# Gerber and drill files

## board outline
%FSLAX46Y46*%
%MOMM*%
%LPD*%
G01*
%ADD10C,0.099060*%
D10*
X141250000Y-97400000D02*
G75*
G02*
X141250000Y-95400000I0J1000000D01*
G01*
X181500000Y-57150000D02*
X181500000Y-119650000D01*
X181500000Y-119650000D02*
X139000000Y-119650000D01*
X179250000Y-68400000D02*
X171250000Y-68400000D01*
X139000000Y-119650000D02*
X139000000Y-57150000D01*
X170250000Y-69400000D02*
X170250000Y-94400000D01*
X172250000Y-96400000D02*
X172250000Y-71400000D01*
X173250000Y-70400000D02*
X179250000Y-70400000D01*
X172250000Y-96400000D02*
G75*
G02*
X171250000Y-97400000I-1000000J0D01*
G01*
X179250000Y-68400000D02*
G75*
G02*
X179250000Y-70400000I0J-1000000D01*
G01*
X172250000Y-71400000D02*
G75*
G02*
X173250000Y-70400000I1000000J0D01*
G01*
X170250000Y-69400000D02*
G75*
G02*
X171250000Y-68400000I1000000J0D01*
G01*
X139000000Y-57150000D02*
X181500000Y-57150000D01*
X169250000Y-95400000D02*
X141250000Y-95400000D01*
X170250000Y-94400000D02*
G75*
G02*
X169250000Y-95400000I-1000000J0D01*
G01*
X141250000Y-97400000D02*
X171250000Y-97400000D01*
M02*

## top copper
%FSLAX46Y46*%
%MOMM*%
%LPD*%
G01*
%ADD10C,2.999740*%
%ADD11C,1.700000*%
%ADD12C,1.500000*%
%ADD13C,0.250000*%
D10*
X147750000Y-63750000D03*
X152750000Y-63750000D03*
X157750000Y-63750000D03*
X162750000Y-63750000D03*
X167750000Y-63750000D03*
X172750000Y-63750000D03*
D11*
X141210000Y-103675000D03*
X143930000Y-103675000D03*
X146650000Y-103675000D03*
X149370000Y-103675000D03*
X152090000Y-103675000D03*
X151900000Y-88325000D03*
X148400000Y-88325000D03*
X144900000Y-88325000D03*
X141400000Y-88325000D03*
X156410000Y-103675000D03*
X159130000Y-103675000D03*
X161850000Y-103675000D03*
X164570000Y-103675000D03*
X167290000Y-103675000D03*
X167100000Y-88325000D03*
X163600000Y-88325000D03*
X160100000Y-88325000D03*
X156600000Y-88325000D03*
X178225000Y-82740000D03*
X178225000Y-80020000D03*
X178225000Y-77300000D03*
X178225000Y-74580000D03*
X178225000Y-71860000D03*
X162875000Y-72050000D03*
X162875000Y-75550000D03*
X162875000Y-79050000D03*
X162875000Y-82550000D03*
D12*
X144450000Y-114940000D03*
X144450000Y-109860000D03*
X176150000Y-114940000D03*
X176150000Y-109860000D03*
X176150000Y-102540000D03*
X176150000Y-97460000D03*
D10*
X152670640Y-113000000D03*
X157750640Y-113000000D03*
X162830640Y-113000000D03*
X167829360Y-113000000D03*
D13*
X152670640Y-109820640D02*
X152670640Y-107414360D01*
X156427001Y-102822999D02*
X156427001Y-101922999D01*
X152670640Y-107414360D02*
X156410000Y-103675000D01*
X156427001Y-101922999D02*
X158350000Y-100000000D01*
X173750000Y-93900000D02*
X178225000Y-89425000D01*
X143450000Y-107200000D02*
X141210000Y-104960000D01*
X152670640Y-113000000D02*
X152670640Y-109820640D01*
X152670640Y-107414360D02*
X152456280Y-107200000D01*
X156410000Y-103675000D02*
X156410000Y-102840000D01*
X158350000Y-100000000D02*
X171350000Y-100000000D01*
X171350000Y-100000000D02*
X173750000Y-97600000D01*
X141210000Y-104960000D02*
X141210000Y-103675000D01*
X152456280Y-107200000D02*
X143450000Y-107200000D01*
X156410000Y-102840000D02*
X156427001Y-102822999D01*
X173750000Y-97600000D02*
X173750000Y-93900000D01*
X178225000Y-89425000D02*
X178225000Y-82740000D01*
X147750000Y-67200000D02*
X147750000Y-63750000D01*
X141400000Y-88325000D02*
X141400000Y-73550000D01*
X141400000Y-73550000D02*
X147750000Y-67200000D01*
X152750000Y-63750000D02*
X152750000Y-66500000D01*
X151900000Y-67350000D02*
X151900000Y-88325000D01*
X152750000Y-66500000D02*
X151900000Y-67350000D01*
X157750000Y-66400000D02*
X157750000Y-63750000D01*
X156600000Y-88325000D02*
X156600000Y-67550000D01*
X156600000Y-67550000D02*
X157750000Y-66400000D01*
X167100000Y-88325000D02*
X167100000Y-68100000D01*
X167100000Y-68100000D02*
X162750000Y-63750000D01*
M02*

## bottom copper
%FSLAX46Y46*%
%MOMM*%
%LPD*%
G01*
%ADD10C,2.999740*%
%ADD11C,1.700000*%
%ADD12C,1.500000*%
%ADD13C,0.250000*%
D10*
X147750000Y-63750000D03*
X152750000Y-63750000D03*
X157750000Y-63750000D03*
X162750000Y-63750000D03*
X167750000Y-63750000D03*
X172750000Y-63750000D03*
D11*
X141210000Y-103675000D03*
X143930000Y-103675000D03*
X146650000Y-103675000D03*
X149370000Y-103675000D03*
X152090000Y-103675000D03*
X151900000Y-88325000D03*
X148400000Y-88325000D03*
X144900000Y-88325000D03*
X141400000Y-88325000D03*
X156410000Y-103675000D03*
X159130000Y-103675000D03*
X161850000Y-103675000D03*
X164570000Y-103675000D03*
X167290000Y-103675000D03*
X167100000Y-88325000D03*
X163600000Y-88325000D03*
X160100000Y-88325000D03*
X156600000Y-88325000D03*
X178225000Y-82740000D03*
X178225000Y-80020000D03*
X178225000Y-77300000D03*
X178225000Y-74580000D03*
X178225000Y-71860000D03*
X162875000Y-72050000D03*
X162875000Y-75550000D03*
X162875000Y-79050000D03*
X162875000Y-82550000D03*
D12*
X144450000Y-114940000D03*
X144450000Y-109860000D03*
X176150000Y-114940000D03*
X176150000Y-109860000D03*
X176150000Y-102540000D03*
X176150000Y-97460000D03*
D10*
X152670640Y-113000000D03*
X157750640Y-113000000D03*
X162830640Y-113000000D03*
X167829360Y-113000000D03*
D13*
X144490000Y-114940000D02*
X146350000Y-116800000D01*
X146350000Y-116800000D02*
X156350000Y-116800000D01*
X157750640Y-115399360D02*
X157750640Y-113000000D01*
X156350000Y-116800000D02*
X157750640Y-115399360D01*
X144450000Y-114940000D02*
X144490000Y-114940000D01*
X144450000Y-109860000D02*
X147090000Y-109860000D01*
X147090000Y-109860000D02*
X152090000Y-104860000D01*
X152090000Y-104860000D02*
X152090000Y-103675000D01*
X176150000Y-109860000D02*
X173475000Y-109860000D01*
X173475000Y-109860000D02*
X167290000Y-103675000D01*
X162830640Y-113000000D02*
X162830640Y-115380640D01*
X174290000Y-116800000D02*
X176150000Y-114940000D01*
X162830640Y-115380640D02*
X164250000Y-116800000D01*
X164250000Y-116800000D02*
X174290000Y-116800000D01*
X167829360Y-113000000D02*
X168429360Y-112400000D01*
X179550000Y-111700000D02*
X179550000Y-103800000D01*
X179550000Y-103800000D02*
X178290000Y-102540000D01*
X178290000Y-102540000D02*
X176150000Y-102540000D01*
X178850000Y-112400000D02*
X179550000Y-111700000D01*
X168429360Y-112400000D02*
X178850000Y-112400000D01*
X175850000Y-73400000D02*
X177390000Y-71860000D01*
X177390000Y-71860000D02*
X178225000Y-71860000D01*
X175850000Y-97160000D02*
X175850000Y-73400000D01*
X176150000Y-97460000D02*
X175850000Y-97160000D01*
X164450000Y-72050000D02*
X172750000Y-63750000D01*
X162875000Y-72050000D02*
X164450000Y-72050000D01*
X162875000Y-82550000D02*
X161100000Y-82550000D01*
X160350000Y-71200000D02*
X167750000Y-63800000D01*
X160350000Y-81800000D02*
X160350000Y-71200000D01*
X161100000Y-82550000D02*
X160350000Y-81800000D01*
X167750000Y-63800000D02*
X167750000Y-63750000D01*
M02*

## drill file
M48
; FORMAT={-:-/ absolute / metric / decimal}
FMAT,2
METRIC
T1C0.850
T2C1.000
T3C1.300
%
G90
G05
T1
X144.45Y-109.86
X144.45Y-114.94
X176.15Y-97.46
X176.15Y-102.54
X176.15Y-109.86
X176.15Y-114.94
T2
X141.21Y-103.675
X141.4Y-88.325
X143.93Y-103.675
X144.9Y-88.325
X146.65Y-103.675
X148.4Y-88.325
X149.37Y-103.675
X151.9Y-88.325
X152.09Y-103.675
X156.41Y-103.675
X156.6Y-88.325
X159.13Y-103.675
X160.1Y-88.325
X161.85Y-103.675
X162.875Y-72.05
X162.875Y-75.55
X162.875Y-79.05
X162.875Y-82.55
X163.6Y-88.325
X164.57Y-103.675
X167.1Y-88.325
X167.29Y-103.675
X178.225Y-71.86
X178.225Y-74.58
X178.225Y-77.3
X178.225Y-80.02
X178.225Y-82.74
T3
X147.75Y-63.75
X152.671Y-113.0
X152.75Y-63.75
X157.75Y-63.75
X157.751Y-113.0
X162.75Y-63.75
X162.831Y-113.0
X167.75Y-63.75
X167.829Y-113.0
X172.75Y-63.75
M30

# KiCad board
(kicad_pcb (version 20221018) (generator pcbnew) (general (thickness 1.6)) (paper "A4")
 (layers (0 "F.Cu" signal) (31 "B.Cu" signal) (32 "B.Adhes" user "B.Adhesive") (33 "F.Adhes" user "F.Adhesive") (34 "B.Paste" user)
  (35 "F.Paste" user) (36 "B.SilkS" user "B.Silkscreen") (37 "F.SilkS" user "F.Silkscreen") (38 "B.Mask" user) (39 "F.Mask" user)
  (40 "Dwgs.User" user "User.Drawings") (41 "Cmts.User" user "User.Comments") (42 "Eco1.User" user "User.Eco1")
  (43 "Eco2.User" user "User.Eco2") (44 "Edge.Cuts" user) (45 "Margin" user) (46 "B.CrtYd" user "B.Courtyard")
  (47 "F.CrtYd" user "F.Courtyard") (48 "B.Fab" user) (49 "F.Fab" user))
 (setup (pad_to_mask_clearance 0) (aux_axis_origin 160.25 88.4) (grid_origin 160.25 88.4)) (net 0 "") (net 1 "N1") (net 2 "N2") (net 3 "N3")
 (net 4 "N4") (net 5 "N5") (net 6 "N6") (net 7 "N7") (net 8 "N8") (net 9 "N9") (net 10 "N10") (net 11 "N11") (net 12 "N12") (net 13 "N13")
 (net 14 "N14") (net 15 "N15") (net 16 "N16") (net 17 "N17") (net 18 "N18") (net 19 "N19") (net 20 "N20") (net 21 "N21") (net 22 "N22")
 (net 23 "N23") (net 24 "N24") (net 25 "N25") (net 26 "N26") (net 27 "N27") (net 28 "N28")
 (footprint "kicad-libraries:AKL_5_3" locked (layer "F.Cu") (at 152.75 63.75)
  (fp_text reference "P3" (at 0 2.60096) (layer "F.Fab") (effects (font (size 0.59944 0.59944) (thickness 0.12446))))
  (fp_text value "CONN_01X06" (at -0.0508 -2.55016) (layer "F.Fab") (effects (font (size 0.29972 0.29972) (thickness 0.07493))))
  (pad "1" thru_hole circle locked (at -5 0) (size 2.99974 2.99974) (drill 1.30048) (layers "*.Cu" "*.Mask" "F.SilkS") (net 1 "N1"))
  (pad "2" thru_hole circle locked (at 0 0) (size 2.99974 2.99974) (drill 1.30048) (layers "*.Cu" "*.Mask" "F.SilkS") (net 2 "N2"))
  (pad "3" thru_hole circle locked (at 5 0) (size 2.99974 2.99974) (drill 1.30048) (layers "*.Cu" "*.Mask" "F.SilkS") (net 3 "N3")))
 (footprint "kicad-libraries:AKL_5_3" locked (layer "F.Cu") (at 167.75 63.75)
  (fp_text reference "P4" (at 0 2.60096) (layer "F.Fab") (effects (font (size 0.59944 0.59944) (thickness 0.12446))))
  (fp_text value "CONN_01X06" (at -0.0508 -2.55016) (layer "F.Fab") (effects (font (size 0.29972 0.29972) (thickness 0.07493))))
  (pad "1" thru_hole circle locked (at -5 0) (size 2.99974 2.99974) (drill 1.30048) (layers "*.Cu" "*.Mask" "F.SilkS") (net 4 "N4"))
  (pad "2" thru_hole circle locked (at 0 0) (size 2.99974 2.99974) (drill 1.30048) (layers "*.Cu" "*.Mask" "F.SilkS") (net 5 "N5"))
  (pad "3" thru_hole circle locked (at 5 0) (size 2.99974 2.99974) (drill 1.30048) (layers "*.Cu" "*.Mask" "F.SilkS") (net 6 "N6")))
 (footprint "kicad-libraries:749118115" (layer "F.Cu") (at 146.65 96)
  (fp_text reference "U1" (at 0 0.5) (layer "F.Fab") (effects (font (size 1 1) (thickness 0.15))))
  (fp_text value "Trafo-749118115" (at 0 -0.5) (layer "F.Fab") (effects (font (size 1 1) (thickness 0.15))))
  (pad "1" thru_hole circle (at -5.44 7.675) (size 1.7 1.7) (drill 1) (layers "*.Cu" "*.Mask") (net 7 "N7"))
  (pad "2" thru_hole circle (at -2.72 7.675) (size 1.7 1.7) (drill 1) (layers "*.Cu" "*.Mask") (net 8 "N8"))
  (pad "3" thru_hole circle (at 0 7.675) (size 1.7 1.7) (drill 1) (layers "*.Cu" "*.Mask") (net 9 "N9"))
  (pad "4" thru_hole circle (at 2.72 7.675) (size 1.7 1.7) (drill 1) (layers "*.Cu" "*.Mask") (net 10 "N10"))
  (pad "5" thru_hole circle (at 5.44 7.675) (size 1.7 1.7) (drill 1) (layers "*.Cu" "*.Mask") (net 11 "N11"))
  (pad "6" thru_hole circle (at 5.25 -7.675) (size 1.7 1.7) (drill 1) (layers "*.Cu" "*.Mask") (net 2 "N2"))
  (pad "7" thru_hole circle (at 1.75 -7.675) (size 1.7 1.7) (drill 1) (layers "*.Cu" "*.Mask") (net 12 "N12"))
  (pad "8" thru_hole circle (at -1.75 -7.675) (size 1.7 1.7) (drill 1) (layers "*.Cu" "*.Mask") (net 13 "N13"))
  (pad "9" thru_hole circle (at -5.25 -7.675) (size 1.7 1.7) (drill 1) (layers "*.Cu" "*.Mask") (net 1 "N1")))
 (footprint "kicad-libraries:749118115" (layer "F.Cu") (at 161.85 96)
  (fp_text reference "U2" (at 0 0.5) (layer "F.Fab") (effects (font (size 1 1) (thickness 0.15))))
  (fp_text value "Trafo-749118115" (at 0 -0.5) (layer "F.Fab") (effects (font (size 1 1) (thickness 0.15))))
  (pad "1" thru_hole circle (at -5.44 7.675) (size 1.7 1.7) (drill 1) (layers "*.Cu" "*.Mask") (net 7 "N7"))
  (pad "2" thru_hole circle (at -2.72 7.675) (size 1.7 1.7) (drill 1) (layers "*.Cu" "*.Mask") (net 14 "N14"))
  (pad "3" thru_hole circle (at 0 7.675) (size 1.7 1.7) (drill 1) (layers "*.Cu" "*.Mask") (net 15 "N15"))
  (pad "4" thru_hole circle (at 2.72 7.675) (size 1.7 1.7) (drill 1) (layers "*.Cu" "*.Mask") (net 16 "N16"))
  (pad "5" thru_hole circle (at 5.44 7.675) (size 1.7 1.7) (drill 1) (layers "*.Cu" "*.Mask") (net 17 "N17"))
  (pad "6" thru_hole circle (at 5.25 -7.675) (size 1.7 1.7) (drill 1) (layers "*.Cu" "*.Mask") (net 4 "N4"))
  (pad "7" thru_hole circle (at 1.75 -7.675) (size 1.7 1.7) (drill 1) (layers "*.Cu" "*.Mask") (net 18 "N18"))
  (pad "8" thru_hole circle (at -1.75 -7.675) (size 1.7 1.7) (drill 1) (layers "*.Cu" "*.Mask") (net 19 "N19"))
  (pad "9" thru_hole circle (at -5.25 -7.675) (size 1.7 1.7) (drill 1) (layers "*.Cu" "*.Mask") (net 3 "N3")))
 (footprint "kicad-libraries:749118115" (layer "F.Cu") (at 170.55 77.3 90)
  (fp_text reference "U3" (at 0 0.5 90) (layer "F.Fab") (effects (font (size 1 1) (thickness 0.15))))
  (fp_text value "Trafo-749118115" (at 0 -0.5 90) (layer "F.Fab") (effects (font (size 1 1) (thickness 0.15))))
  (pad "1" thru_hole circle (at -5.44 7.675 90) (size 1.7 1.7) (drill 1) (layers "*.Cu" "*.Mask") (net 7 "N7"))
  (pad "2" thru_hole circle (at -2.72 7.675 90) (size 1.7 1.7) (drill 1) (layers "*.Cu" "*.Mask") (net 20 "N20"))
  (pad "3" thru_hole circle (at 0 7.675 90) (size 1.7 1.7) (drill 1) (layers "*.Cu" "*.Mask") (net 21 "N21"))
  (pad "4" thru_hole circle (at 2.72 7.675 90) (size 1.7 1.7) (drill 1) (layers "*.Cu" "*.Mask") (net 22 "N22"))
  (pad "5" thru_hole circle (at 5.44 7.675 90) (size 1.7 1.7) (drill 1) (layers "*.Cu" "*.Mask") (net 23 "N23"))
  (pad "6" thru_hole circle (at 5.25 -7.675 90) (size 1.7 1.7) (drill 1) (layers "*.Cu" "*.Mask") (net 6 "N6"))
  (pad "7" thru_hole circle (at 1.75 -7.675 90) (size 1.7 1.7) (drill 1) (layers "*.Cu" "*.Mask") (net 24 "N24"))
  (pad "8" thru_hole circle (at -1.75 -7.675 90) (size 1.7 1.7) (drill 1) (layers "*.Cu" "*.Mask") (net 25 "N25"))
  (pad "9" thru_hole circle (at -5.25 -7.675 90) (size 1.7 1.7) (drill 1) (layers "*.Cu" "*.Mask") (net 5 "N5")))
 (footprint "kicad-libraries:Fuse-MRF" (layer "F.Cu") (at 144.45 112.4 90)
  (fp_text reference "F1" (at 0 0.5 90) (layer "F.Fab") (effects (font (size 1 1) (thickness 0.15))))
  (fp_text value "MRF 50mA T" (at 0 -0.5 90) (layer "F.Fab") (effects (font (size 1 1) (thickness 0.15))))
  (pad "1" thru_hole circle (at -2.54 0 90) (size 1.5 1.5) (drill 0.85) (layers "*.Cu" "*.Mask") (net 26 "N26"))
  (pad "2" thru_hole circle (at 2.54 0 90) (size 1.5 1.5) (drill 0.85) (layers "*.Cu" "*.Mask") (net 11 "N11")))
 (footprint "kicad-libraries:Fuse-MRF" (layer "F.Cu") (at 176.15 112.4 90)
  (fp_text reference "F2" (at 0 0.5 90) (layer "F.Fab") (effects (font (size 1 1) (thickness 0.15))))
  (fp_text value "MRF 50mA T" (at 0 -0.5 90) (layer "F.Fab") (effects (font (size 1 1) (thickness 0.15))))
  (pad "1" thru_hole circle (at -2.54 0 90) (size 1.5 1.5) (drill 0.85) (layers "*.Cu" "*.Mask") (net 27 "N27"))
  (pad "2" thru_hole circle (at 2.54 0 90) (size 1.5 1.5) (drill 0.85) (layers "*.Cu" "*.Mask") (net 17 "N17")))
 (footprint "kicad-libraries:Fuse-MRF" (layer "F.Cu") (at 176.15 100 90)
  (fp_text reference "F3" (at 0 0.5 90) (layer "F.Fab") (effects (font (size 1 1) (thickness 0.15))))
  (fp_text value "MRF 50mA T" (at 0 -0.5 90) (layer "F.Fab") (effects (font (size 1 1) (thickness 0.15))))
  (pad "1" thru_hole circle (at -2.54 0 90) (size 1.5 1.5) (drill 0.85) (layers "*.Cu" "*.Mask") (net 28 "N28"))
  (pad "2" thru_hole circle (at 2.54 0 90) (size 1.5 1.5) (drill 0.85) (layers "*.Cu" "*.Mask") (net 23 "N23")))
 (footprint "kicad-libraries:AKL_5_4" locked (layer "F.Cu") (at 160.25 113 180)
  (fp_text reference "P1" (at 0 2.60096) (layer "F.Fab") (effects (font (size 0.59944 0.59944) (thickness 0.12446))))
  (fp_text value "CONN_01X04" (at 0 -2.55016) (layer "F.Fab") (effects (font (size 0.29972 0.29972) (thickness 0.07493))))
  (pad "1" thru_hole circle locked (at 7.57936 0 180) (size 2.99974 2.99974) (drill 1.30048) (layers "*.Cu" "*.Mask" "F.SilkS") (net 7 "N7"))
  (pad "2" thru_hole circle locked (at 2.49936 0 180) (size 2.99974 2.99974) (drill 1.30048) (layers "*.Cu" "*.Mask" "F.SilkS")
   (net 26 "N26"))
  (pad "3" thru_hole circle locked (at -2.58064 0 180) (size 2.99974 2.99974) (drill 1.30048) (layers "*.Cu" "*.Mask" "F.SilkS")
   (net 27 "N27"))
  (pad "4" thru_hole circle locked (at -7.57936 0 180) (size 2.99974 2.99974) (drill 1.30048) (layers "*.Cu" "*.Mask" "F.SilkS")
   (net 28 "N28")))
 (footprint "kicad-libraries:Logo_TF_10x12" (layer "F.Cu") (at 149.25 74.4)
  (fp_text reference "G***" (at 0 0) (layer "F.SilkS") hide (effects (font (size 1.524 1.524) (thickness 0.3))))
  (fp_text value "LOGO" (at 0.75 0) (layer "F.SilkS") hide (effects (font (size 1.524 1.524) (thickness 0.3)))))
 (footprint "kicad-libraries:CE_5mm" (layer "B.Cu") (at 148.95 73.1 180)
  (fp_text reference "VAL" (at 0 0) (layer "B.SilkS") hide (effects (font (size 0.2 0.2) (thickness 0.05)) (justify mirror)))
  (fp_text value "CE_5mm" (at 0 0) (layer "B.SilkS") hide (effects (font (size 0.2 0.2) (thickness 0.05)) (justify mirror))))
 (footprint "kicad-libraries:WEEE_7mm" (layer "B.Cu") (at 148.85 80.5 180)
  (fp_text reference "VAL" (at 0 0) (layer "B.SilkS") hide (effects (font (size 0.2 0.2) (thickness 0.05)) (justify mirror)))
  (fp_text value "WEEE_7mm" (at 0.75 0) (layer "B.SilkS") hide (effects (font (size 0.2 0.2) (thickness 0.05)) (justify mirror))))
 (gr_arc (start 141.25 97.4) (mid 140.25 96.4) (end 141.25 95.4) (stroke (width 0.09906) (type solid)) (layer "Edge.Cuts"))
 (gr_line (start 181.5 57.15) (end 181.5 119.65) (stroke (width 0.09906) (type solid)) (layer "Edge.Cuts"))
 (gr_line (start 181.5 119.65) (end 139 119.65) (stroke (width 0.09906) (type solid)) (layer "Edge.Cuts"))
 (gr_line (start 179.25 68.4) (end 171.25 68.4) (stroke (width 0.09906) (type solid)) (layer "Edge.Cuts"))
 (gr_line (start 139 119.65) (end 139 57.15) (stroke (width 0.09906) (type solid)) (layer "Edge.Cuts"))
 (gr_line (start 170.25 69.4) (end 170.25 94.4) (stroke (width 0.09906) (type solid)) (layer "Edge.Cuts"))
 (gr_line (start 172.25 96.4) (end 172.25 71.4) (stroke (width 0.09906) (type solid)) (layer "Edge.Cuts"))
 (gr_line (start 173.25 70.4) (end 179.25 70.4) (stroke (width 0.09906) (type solid)) (layer "Edge.Cuts"))
 (gr_arc (start 172.25 96.4) (mid 171.957107 97.107107) (end 171.25 97.4) (stroke (width 0.09906) (type solid)) (layer "Edge.Cuts"))
 (gr_arc (start 179.25 68.4) (mid 180.25 69.4) (end 179.25 70.4) (stroke (width 0.09906) (type solid)) (layer "Edge.Cuts"))
 (gr_arc (start 172.25 71.4) (mid 172.542893 70.692893) (end 173.25 70.4) (stroke (width 0.09906) (type solid)) (layer "Edge.Cuts"))
 (gr_arc (start 170.25 69.4) (mid 170.542893 68.692893) (end 171.25 68.4) (stroke (width 0.09906) (type solid)) (layer "Edge.Cuts"))
 (gr_line (start 139 57.15) (end 181.5 57.15) (stroke (width 0.09906) (type solid)) (layer "Edge.Cuts"))
 (gr_line (start 169.25 95.4) (end 141.25 95.4) (stroke (width 0.09906) (type solid)) (layer "Edge.Cuts"))
 (gr_arc (start 170.25 94.4) (mid 169.957107 95.107107) (end 169.25 95.4) (stroke (width 0.09906) (type solid)) (layer "Edge.Cuts"))
 (gr_line (start 141.25 97.4) (end 171.25 97.4) (stroke (width 0.09906) (type solid)) (layer "Edge.Cuts"))
 (segment (start 144.49 114.94) (end 146.35 116.8) (width 0.25) (layer "B.Cu") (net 26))
 (segment (start 146.35 116.8) (end 156.35 116.8) (width 0.25) (layer "B.Cu") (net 26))
 (segment (start 157.75064 115.39936) (end 157.75064 113) (width 0.25) (layer "B.Cu") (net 26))
 (segment (start 156.35 116.8) (end 157.75064 115.39936) (width 0.25) (layer "B.Cu") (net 26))
 (segment (start 144.45 114.94) (end 144.49 114.94) (width 0.25) (layer "B.Cu") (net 26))
 (segment (start 144.45 109.86) (end 147.09 109.86) (width 0.25) (layer "B.Cu") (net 11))
 (segment (start 147.09 109.86) (end 152.09 104.86) (width 0.25) (layer "B.Cu") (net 11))
 (segment (start 152.09 104.86) (end 152.09 103.675) (width 0.25) (layer "B.Cu") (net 11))
 (segment (start 176.15 109.86) (end 173.475 109.86) (width 0.25) (layer "B.Cu") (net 17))
 (segment (start 173.475 109.86) (end 167.29 103.675) (width 0.25) (layer "B.Cu") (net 17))
 (segment (start 162.83064 113) (end 162.83064 115.38064) (width 0.25) (layer "B.Cu") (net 27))
 (segment (start 174.29 116.8) (end 176.15 114.94) (width 0.25) (layer "B.Cu") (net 27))
 (segment (start 162.83064 115.38064) (end 164.25 116.8) (width 0.25) (layer "B.Cu") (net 27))
 (segment (start 164.25 116.8) (end 174.29 116.8) (width 0.25) (layer "B.Cu") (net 27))
 (segment (start 167.82936 113) (end 168.42936 112.4) (width 0.25) (layer "B.Cu") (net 28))
 (segment (start 179.55 111.7) (end 179.55 103.8) (width 0.25) (layer "B.Cu") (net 28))
 (segment (start 179.55 103.8) (end 178.29 102.54) (width 0.25) (layer "B.Cu") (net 28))
 (segment (start 178.29 102.54) (end 176.15 102.54) (width 0.25) (layer "B.Cu") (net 28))
 (segment (start 178.85 112.4) (end 179.55 111.7) (width 0.25) (layer "B.Cu") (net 28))
 (segment (start 168.42936 112.4) (end 178.85 112.4) (width 0.25) (layer "B.Cu") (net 28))
 (segment (start 175.85 73.4) (end 177.39 71.86) (width 0.25) (layer "B.Cu") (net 23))
 (segment (start 177.39 71.86) (end 178.225 71.86) (width 0.25) (layer "B.Cu") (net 23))
 (segment (start 175.85 97.16) (end 175.85 73.4) (width 0.25) (layer "B.Cu") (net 23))
 (segment (start 176.15 97.46) (end 175.85 97.16) (width 0.25) (layer "B.Cu") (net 23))
 (segment (start 152.67064 109.82064) (end 152.67064 107.41436) (width 0.25) (layer "F.Cu") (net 7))
 (segment (start 156.427001 102.822999) (end 156.427001 101.922999) (width 0.25) (layer "F.Cu") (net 7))
 (segment (start 152.67064 107.41436) (end 156.41 103.675) (width 0.25) (layer "F.Cu") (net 7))
 (segment (start 156.427001 101.922999) (end 158.35 100) (width 0.25) (layer "F.Cu") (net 7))
 (segment (start 173.75 93.9) (end 178.225 89.425) (width 0.25) (layer "F.Cu") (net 7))
 (segment (start 143.45 107.2) (end 141.21 104.96) (width 0.25) (layer "F.Cu") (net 7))
 (segment (start 152.67064 113) (end 152.67064 109.82064) (width 0.25) (layer "F.Cu") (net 7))
 (segment (start 152.67064 107.41436) (end 152.45628 107.2) (width 0.25) (layer "F.Cu") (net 7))
 (segment (start 156.41 103.675) (end 156.41 102.84) (width 0.25) (layer "F.Cu") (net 7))
 (segment (start 158.35 100) (end 171.35 100) (width 0.25) (layer "F.Cu") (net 7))
 (segment (start 171.35 100) (end 173.75 97.6) (width 0.25) (layer "F.Cu") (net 7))
 (segment (start 141.21 104.96) (end 141.21 103.675) (width 0.25) (layer "F.Cu") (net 7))
 (segment (start 152.45628 107.2) (end 143.45 107.2) (width 0.25) (layer "F.Cu") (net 7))
 (segment (start 156.41 102.84) (end 156.427001 102.822999) (width 0.25) (layer "F.Cu") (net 7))
 (segment (start 173.75 97.6) (end 173.75 93.9) (width 0.25) (layer "F.Cu") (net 7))
 (segment (start 178.225 89.425) (end 178.225 82.74) (width 0.25) (layer "F.Cu") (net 7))
 (segment (start 147.75 67.2) (end 147.75 63.75) (width 0.25) (layer "F.Cu") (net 1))
 (segment (start 141.4 88.325) (end 141.4 73.55) (width 0.25) (layer "F.Cu") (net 1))
 (segment (start 141.4 73.55) (end 147.75 67.2) (width 0.25) (layer "F.Cu") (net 1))
 (segment (start 152.75 63.75) (end 152.75 66.5) (width 0.25) (layer "F.Cu") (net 2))
 (segment (start 151.9 67.35) (end 151.9 88.325) (width 0.25) (layer "F.Cu") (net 2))
 (segment (start 152.75 66.5) (end 151.9 67.35) (width 0.25) (layer "F.Cu") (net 2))
 (segment (start 157.75 66.4) (end 157.75 63.75) (width 0.25) (layer "F.Cu") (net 3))
 (segment (start 156.6 88.325) (end 156.6 67.55) (width 0.25) (layer "F.Cu") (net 3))
 (segment (start 156.6 67.55) (end 157.75 66.4) (width 0.25) (layer "F.Cu") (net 3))
 (segment (start 164.45 72.05) (end 172.75 63.75) (width 0.25) (layer "B.Cu") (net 6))
 (segment (start 162.875 72.05) (end 164.45 72.05) (width 0.25) (layer "B.Cu") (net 6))
 (segment (start 162.875 82.55) (end 161.1 82.55) (width 0.25) (layer "B.Cu") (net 5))
 (segment (start 160.35 71.2) (end 167.75 63.8) (width 0.25) (layer "B.Cu") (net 5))
 (segment (start 160.35 81.8) (end 160.35 71.2) (width 0.25) (layer "B.Cu") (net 5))
 (segment (start 161.1 82.55) (end 160.35 81.8) (width 0.25) (layer "B.Cu") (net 5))
 (segment (start 167.75 63.8) (end 167.75 63.75) (width 0.25) (layer "B.Cu") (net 5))
 (segment (start 167.1 88.325) (end 167.1 68.1) (width 0.25) (layer "F.Cu") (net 4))
 (segment (start 167.1 68.1) (end 162.75 63.75) (width 0.25) (layer "F.Cu") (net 4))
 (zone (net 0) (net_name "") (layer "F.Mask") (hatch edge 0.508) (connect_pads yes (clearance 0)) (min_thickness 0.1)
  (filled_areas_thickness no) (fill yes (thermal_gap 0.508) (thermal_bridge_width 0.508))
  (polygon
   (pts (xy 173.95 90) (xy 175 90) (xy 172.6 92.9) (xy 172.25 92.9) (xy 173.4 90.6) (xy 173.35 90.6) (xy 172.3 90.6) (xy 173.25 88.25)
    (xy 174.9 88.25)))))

